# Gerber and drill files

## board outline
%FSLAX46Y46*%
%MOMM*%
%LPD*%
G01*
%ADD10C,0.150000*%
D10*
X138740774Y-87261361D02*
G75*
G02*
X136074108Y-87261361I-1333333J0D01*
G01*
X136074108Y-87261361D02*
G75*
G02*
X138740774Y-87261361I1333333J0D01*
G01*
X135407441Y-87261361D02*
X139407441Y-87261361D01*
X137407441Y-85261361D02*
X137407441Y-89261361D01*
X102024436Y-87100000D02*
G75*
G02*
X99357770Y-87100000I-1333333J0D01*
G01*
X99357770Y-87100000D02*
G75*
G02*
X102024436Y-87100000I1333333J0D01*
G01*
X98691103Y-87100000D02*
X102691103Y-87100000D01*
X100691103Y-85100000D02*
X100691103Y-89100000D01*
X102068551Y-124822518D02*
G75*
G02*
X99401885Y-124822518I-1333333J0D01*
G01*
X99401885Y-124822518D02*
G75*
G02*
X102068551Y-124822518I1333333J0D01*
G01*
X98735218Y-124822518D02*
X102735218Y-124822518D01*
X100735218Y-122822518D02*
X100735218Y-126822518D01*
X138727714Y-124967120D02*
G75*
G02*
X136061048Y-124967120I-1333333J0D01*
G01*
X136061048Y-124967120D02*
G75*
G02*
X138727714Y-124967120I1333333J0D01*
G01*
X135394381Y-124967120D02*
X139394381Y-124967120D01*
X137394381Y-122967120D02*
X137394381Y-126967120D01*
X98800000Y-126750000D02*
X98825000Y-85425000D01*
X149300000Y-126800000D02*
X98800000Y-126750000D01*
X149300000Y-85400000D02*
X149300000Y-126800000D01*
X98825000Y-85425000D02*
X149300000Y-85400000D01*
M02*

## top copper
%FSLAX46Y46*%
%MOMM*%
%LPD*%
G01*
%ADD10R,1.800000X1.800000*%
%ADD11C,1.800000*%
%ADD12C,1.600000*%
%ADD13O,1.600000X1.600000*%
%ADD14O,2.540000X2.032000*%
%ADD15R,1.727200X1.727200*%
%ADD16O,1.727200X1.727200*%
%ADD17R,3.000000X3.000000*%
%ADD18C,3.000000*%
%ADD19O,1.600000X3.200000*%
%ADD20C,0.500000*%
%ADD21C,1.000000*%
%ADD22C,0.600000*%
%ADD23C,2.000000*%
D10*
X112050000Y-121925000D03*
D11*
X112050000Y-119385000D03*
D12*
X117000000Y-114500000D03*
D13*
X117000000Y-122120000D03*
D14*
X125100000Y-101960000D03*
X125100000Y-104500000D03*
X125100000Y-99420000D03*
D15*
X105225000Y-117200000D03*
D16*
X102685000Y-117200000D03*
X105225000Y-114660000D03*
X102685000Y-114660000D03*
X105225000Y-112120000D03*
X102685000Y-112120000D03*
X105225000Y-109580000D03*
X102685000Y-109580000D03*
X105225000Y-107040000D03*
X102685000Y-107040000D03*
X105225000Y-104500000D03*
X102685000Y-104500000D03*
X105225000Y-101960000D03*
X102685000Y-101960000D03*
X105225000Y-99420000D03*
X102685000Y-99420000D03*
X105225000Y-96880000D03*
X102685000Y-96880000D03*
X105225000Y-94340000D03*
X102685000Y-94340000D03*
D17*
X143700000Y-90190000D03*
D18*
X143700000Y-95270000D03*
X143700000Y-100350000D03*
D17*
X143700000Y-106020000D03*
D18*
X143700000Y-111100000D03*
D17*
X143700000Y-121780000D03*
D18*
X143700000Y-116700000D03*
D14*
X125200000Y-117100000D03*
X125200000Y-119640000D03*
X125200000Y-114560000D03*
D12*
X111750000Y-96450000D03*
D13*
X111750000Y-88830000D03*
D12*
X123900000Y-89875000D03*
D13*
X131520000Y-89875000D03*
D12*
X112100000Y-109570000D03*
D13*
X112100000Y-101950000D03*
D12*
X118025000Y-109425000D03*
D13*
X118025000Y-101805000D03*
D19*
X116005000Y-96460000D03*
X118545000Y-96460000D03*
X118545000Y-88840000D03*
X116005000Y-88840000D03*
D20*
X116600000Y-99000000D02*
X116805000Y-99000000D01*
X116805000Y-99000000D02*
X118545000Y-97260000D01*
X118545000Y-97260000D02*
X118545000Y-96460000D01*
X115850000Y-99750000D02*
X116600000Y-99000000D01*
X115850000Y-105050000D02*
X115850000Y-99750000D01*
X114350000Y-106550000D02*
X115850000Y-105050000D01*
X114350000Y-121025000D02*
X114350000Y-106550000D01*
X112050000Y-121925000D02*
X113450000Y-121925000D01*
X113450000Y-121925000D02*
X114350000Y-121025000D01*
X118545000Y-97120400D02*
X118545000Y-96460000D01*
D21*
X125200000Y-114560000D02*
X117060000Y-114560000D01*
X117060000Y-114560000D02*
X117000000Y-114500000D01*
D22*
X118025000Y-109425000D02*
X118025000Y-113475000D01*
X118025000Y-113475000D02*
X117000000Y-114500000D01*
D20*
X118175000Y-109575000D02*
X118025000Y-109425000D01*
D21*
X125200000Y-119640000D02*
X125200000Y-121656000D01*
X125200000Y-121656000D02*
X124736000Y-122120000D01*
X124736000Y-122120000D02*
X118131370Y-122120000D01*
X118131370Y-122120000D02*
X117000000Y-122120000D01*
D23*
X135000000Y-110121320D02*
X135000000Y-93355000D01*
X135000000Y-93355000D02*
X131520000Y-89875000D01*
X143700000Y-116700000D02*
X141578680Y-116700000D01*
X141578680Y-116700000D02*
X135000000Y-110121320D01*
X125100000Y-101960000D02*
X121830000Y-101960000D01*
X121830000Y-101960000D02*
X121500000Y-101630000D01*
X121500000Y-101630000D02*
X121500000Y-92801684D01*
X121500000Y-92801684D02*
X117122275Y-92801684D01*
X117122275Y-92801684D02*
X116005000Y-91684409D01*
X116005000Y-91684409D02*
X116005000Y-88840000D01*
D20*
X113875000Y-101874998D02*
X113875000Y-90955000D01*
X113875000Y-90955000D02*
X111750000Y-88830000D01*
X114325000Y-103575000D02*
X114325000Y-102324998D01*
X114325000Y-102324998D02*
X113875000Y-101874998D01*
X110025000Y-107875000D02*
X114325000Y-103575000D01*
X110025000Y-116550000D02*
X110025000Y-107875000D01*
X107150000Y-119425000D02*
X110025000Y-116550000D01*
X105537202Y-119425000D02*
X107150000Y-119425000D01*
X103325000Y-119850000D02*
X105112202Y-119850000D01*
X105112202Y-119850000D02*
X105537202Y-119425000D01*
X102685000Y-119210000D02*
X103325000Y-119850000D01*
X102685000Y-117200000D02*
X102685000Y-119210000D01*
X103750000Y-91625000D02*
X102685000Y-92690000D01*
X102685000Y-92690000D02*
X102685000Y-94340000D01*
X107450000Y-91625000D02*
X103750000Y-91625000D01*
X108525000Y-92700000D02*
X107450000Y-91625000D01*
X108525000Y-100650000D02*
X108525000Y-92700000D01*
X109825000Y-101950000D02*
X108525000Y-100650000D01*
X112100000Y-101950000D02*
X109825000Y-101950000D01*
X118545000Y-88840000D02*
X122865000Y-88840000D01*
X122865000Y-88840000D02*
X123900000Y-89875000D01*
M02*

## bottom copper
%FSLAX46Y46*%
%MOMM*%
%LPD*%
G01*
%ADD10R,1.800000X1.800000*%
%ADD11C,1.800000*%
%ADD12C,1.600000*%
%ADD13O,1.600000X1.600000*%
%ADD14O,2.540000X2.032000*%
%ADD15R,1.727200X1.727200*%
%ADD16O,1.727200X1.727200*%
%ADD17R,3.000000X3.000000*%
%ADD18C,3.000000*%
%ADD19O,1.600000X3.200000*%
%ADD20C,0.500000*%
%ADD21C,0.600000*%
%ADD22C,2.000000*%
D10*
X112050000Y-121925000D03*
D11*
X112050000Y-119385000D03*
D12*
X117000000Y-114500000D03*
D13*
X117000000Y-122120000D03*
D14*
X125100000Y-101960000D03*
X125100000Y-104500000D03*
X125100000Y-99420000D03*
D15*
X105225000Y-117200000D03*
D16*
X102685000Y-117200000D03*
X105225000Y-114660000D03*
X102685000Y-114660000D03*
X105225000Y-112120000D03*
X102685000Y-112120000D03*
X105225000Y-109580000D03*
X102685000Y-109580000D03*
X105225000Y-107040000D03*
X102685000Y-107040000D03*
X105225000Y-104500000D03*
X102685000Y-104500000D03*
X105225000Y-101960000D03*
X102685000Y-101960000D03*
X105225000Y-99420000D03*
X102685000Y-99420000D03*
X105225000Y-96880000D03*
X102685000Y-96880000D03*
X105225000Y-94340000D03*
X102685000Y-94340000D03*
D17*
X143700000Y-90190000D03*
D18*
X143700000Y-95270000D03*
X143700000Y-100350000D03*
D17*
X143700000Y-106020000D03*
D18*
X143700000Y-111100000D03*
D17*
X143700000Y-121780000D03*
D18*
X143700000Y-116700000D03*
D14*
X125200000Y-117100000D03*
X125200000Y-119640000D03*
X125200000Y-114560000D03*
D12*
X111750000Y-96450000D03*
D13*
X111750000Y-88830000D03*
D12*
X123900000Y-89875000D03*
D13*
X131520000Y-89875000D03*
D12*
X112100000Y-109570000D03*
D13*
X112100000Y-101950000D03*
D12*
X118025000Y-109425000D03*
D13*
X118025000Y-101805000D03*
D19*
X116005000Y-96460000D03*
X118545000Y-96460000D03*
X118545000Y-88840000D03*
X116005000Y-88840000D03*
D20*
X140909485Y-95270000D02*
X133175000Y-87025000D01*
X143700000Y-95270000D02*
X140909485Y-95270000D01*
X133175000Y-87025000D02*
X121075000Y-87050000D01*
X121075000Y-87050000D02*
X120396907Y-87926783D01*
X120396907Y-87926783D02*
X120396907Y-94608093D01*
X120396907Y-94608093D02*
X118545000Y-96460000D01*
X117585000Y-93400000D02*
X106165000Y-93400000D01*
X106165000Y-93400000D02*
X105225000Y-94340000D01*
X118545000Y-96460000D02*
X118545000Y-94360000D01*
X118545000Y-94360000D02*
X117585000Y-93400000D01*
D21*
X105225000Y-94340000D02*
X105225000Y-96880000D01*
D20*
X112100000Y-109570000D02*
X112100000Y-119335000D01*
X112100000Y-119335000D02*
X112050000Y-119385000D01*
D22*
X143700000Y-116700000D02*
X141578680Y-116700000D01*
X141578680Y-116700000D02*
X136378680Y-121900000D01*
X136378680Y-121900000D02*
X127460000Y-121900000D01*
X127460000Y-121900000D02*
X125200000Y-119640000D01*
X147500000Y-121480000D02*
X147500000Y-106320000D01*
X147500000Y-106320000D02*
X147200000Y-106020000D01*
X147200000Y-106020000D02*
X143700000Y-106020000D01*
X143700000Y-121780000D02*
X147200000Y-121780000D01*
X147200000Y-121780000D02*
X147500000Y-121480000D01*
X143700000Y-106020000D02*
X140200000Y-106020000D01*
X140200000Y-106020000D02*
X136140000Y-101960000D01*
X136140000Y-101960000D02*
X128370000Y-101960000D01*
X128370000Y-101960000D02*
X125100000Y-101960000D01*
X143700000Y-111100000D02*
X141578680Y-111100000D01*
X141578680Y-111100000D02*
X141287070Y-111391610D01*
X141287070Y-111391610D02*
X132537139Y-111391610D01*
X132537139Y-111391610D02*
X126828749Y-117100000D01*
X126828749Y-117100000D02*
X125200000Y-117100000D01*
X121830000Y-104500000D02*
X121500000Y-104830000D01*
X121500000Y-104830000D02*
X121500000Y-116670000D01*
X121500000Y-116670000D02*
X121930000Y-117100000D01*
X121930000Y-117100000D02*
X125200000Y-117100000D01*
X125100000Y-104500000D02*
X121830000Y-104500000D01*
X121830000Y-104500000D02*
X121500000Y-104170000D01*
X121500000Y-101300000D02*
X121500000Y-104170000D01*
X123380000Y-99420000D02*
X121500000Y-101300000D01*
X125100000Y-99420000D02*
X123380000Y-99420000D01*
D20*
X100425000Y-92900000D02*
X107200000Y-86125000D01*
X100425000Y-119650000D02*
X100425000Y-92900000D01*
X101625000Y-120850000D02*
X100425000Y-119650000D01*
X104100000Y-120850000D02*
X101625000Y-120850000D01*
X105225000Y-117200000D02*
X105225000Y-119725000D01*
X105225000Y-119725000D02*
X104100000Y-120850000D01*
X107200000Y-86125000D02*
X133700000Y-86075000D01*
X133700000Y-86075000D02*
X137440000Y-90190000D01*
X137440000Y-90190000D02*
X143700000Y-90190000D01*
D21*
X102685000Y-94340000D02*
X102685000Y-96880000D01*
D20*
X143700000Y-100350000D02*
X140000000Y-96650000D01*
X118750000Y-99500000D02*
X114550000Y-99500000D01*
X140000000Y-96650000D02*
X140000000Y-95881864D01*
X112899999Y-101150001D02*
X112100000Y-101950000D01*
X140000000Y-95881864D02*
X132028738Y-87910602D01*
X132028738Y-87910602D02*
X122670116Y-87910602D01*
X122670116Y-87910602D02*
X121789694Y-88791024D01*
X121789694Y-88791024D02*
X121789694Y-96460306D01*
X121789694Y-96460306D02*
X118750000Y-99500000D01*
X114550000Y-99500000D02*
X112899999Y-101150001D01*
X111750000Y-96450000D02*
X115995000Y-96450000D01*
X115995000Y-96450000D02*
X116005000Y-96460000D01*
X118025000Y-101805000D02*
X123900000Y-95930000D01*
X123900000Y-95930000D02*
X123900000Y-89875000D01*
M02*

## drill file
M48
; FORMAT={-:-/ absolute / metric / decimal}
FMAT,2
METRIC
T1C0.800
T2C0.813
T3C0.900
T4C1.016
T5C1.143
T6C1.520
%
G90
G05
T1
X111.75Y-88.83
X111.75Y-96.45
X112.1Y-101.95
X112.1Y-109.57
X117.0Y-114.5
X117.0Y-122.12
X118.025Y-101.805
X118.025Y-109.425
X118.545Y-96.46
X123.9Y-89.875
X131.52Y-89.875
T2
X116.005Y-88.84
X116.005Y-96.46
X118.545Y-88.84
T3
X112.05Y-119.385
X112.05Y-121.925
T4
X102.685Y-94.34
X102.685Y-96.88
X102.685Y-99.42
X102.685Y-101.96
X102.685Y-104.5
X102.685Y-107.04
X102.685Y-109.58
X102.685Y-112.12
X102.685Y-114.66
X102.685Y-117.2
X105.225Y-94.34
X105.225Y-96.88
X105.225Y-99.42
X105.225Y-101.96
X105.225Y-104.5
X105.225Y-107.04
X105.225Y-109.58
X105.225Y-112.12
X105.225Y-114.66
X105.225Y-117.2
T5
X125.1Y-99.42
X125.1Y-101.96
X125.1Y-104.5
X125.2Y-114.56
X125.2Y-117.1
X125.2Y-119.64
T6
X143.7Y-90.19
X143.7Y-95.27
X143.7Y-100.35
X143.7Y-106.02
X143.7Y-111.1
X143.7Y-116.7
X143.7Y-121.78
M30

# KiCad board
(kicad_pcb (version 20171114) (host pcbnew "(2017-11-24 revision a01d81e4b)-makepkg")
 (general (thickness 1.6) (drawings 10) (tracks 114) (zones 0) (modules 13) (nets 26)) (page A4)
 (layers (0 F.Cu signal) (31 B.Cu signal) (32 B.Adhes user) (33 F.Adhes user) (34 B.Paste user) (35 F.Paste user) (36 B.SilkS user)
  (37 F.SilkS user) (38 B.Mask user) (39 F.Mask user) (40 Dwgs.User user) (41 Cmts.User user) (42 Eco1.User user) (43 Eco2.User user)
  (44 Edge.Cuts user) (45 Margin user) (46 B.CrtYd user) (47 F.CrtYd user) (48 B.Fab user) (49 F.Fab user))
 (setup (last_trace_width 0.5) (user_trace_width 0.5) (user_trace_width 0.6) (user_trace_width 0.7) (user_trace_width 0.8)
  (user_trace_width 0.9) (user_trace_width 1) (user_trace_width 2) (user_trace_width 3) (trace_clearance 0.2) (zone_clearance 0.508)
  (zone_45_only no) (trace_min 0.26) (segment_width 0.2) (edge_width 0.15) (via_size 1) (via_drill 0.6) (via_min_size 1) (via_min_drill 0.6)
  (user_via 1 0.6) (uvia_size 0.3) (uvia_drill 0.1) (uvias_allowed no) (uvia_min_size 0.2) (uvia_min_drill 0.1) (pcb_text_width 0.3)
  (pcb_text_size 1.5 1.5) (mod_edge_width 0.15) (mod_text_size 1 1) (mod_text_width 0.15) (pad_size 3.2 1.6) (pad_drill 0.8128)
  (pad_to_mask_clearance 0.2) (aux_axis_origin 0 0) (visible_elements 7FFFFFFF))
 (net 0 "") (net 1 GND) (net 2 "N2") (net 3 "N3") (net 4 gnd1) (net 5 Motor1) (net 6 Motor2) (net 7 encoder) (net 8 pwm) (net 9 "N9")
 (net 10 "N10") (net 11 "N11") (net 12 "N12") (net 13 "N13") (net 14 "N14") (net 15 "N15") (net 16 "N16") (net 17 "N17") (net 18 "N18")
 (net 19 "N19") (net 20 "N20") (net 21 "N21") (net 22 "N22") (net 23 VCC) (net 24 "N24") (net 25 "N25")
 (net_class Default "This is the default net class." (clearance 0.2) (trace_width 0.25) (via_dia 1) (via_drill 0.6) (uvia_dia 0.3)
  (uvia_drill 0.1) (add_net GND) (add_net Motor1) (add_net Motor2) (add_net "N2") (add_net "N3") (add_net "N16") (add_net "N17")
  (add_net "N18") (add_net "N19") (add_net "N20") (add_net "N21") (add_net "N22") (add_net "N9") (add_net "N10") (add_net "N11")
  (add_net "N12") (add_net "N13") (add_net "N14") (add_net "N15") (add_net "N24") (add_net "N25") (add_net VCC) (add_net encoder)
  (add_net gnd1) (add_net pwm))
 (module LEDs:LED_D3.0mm (layer F.Cu) (at 112.05 121.925 90)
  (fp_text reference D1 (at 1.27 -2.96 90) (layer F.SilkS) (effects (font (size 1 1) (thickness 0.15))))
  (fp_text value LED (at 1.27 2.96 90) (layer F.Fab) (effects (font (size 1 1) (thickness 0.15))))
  (pad 1 thru_hole rect (at 0 0 90) (size 1.8 1.8) (drill 0.9) (layers *.Cu *.Mask) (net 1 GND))
  (pad 2 thru_hole circle (at 2.54 0 90) (size 1.8 1.8) (drill 0.9) (layers *.Cu *.Mask) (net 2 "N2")))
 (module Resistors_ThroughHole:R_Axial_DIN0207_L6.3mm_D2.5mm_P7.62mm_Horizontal (layer F.Cu) (at 117 114.5 270)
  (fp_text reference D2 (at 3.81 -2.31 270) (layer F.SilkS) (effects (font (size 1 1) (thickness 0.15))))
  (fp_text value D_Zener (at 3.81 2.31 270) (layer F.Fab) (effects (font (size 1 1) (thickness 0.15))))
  (pad 1 thru_hole circle (at 0 0 270) (size 1.6 1.6) (drill 0.8) (layers *.Cu *.Mask) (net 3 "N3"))
  (pad 2 thru_hole oval (at 7.62 0 270) (size 1.6 1.6) (drill 0.8) (layers *.Cu *.Mask) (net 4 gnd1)))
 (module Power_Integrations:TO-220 (layer F.Cu) (at 125.1 101.96 270)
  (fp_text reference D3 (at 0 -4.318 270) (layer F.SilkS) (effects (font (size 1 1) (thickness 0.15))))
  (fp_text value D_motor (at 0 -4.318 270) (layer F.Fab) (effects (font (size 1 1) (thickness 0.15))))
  (pad 2 thru_hole oval (at 0 0 270) (size 2.032 2.54) (drill 1.143) (layers *.Cu *.Mask) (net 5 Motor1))
  (pad 3 thru_hole oval (at 2.54 0 270) (size 2.032 2.54) (drill 1.143) (layers *.Cu *.Mask) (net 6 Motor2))
  (pad 1 thru_hole oval (at -2.54 0 270) (size 2.032 2.54) (drill 1.143) (layers *.Cu *.Mask) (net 6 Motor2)))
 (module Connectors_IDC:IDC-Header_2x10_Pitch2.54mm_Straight (layer F.Cu) (at 105.225 117.2 180)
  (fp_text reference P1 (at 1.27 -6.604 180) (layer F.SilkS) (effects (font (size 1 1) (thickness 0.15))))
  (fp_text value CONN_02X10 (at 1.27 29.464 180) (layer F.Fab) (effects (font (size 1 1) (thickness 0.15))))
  (pad 1 thru_hole rect (at 0 0 180) (size 1.7272 1.7272) (drill 1.016) (layers *.Cu *.Mask) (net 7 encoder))
  (pad 2 thru_hole oval (at 2.54 0 180) (size 1.7272 1.7272) (drill 1.016) (layers *.Cu *.Mask) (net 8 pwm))
  (pad 3 thru_hole oval (at 0 2.54 180) (size 1.7272 1.7272) (drill 1.016) (layers *.Cu *.Mask) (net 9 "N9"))
  (pad 4 thru_hole oval (at 2.54 2.54 180) (size 1.7272 1.7272) (drill 1.016) (layers *.Cu *.Mask) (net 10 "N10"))
  (pad 5 thru_hole oval (at 0 5.08 180) (size 1.7272 1.7272) (drill 1.016) (layers *.Cu *.Mask) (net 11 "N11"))
  (pad 6 thru_hole oval (at 2.54 5.08 180) (size 1.7272 1.7272) (drill 1.016) (layers *.Cu *.Mask) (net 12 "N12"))
  (pad 7 thru_hole oval (at 0 7.62 180) (size 1.7272 1.7272) (drill 1.016) (layers *.Cu *.Mask) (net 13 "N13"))
  (pad 8 thru_hole oval (at 2.54 7.62 180) (size 1.7272 1.7272) (drill 1.016) (layers *.Cu *.Mask) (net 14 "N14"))
  (pad 9 thru_hole oval (at 0 10.16 180) (size 1.7272 1.7272) (drill 1.016) (layers *.Cu *.Mask) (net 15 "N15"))
  (pad 10 thru_hole oval (at 2.54 10.16 180) (size 1.7272 1.7272) (drill 1.016) (layers *.Cu *.Mask) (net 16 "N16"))
  (pad 11 thru_hole oval (at 0 12.7 180) (size 1.7272 1.7272) (drill 1.016) (layers *.Cu *.Mask) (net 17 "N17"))
  (pad 12 thru_hole oval (at 2.54 12.7 180) (size 1.7272 1.7272) (drill 1.016) (layers *.Cu *.Mask) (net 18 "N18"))
  (pad 13 thru_hole oval (at 0 15.24 180) (size 1.7272 1.7272) (drill 1.016) (layers *.Cu *.Mask) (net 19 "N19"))
  (pad 14 thru_hole oval (at 2.54 15.24 180) (size 1.7272 1.7272) (drill 1.016) (layers *.Cu *.Mask) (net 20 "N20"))
  (pad 15 thru_hole oval (at 0 17.78 180) (size 1.7272 1.7272) (drill 1.016) (layers *.Cu *.Mask) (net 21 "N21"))
  (pad 16 thru_hole oval (at 2.54 17.78 180) (size 1.7272 1.7272) (drill 1.016) (layers *.Cu *.Mask) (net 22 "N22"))
  (pad 17 thru_hole oval (at 0 20.32 180) (size 1.7272 1.7272) (drill 1.016) (layers *.Cu *.Mask) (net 1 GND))
  (pad 18 thru_hole oval (at 2.54 20.32 180) (size 1.7272 1.7272) (drill 1.016) (layers *.Cu *.Mask) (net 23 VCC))
  (pad 19 thru_hole oval (at 0 22.86 180) (size 1.7272 1.7272) (drill 1.016) (layers *.Cu *.Mask) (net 1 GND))
  (pad 20 thru_hole oval (at 2.54 22.86 180) (size 1.7272 1.7272) (drill 1.016) (layers *.Cu *.Mask) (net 23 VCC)))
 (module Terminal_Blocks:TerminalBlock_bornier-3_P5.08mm (layer F.Cu) (at 143.7 90.19 270)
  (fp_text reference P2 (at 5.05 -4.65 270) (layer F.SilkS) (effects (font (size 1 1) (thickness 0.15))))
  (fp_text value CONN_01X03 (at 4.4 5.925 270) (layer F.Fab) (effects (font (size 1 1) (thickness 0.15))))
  (pad 1 thru_hole rect (at 0 0 270) (size 3 3) (drill 1.52) (layers *.Cu *.Mask) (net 7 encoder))
  (pad 2 thru_hole circle (at 5.08 0 270) (size 3 3) (drill 1.52) (layers *.Cu *.Mask) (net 1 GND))
  (pad 3 thru_hole circle (at 10.16 0 270) (size 3 3) (drill 1.52) (layers *.Cu *.Mask) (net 23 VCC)))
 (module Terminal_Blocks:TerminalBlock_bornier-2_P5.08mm (layer F.Cu) (at 143.7 106.02 270)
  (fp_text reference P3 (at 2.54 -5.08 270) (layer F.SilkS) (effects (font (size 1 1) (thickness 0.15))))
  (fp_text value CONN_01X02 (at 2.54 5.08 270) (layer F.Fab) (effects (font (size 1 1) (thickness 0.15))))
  (pad 1 thru_hole rect (at 0 0 270) (size 3 3) (drill 1.52) (layers *.Cu *.Mask) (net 5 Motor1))
  (pad 2 thru_hole circle (at 5.08 0 270) (size 3 3) (drill 1.52) (layers *.Cu *.Mask) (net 6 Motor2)))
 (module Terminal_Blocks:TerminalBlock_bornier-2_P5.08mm (layer F.Cu) (at 143.7 121.78 90)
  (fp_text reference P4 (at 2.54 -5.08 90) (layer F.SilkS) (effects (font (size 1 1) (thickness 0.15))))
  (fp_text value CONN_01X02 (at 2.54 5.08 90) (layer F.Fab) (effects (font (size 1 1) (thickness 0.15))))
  (pad 1 thru_hole rect (at 0 0 90) (size 3 3) (drill 1.52) (layers *.Cu *.Mask) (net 5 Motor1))
  (pad 2 thru_hole circle (at 5.08 0 90) (size 3 3) (drill 1.52) (layers *.Cu *.Mask) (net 4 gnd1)))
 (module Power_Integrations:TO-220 (layer F.Cu) (at 125.2 117.1 270)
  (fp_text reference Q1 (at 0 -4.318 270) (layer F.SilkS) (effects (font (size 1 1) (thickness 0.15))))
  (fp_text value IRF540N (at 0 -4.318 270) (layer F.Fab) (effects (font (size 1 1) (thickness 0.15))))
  (pad 2 thru_hole oval (at 0 0 270) (size 2.032 2.54) (drill 1.143) (layers *.Cu *.Mask) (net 6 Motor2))
  (pad 3 thru_hole oval (at 2.54 0 270) (size 2.032 2.54) (drill 1.143) (layers *.Cu *.Mask) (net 4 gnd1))
  (pad 1 thru_hole oval (at -2.54 0 270) (size 2.032 2.54) (drill 1.143) (layers *.Cu *.Mask) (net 3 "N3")))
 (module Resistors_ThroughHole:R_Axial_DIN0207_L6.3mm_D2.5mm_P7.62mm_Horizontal (layer F.Cu) (at 111.75 96.45 90)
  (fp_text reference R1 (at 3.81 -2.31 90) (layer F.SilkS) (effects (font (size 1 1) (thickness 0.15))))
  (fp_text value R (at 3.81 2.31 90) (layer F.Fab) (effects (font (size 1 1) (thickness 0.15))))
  (pad 1 thru_hole circle (at 0 0 90) (size 1.6 1.6) (drill 0.8) (layers *.Cu *.Mask) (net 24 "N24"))
  (pad 2 thru_hole oval (at 7.62 0 90) (size 1.6 1.6) (drill 0.8) (layers *.Cu *.Mask) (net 8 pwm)))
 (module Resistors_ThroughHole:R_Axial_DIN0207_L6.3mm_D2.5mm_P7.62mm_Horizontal (layer F.Cu) (at 123.9 89.875)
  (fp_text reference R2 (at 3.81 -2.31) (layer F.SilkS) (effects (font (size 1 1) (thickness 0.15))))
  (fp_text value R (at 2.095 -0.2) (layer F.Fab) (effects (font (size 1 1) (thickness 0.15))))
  (pad 1 thru_hole circle (at 0 0) (size 1.6 1.6) (drill 0.8) (layers *.Cu *.Mask) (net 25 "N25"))
  (pad 2 thru_hole oval (at 7.62 0) (size 1.6 1.6) (drill 0.8) (layers *.Cu *.Mask) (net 4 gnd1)))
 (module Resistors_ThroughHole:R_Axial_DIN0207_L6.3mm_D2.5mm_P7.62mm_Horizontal (layer F.Cu) (at 112.1 109.57 90)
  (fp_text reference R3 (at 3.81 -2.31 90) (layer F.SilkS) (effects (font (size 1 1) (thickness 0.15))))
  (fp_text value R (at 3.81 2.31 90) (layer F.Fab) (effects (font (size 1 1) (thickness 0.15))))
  (pad 1 thru_hole circle (at 0 0 90) (size 1.6 1.6) (drill 0.8) (layers *.Cu *.Mask) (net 2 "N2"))
  (pad 2 thru_hole oval (at 7.62 0 90) (size 1.6 1.6) (drill 0.8) (layers *.Cu *.Mask) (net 23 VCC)))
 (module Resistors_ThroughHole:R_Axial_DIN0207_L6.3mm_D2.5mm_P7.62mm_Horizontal (layer F.Cu) (at 118.025 109.425 90)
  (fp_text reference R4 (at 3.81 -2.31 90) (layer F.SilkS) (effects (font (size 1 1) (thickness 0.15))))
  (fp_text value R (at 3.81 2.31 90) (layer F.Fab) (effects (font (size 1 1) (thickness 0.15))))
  (pad 1 thru_hole circle (at 0 0 90) (size 1.6 1.6) (drill 0.8) (layers *.Cu *.Mask) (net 3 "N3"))
  (pad 2 thru_hole oval (at 7.62 0 90) (size 1.6 1.6) (drill 0.8) (layers *.Cu *.Mask) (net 25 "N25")))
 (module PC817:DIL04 (layer F.Cu) (at 117.275 92.65) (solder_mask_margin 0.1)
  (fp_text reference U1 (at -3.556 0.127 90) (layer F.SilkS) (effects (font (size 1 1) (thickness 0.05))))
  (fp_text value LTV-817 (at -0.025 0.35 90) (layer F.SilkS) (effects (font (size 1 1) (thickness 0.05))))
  (pad 1 thru_hole oval (at -1.27 3.81 270) (size 3.2 1.6) (drill 0.8128) (layers *.Cu *.Mask F.SilkS) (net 24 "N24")
   (solder_mask_margin 0.2))
  (pad 2 thru_hole oval (at 1.27 3.81 270) (size 3.2 1.6) (drill 0.8) (layers *.Cu *.Mask F.SilkS) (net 1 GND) (solder_mask_margin 0.2))
  (pad 3 thru_hole oval (at 1.27 -3.81 90) (size 3.2 1.6) (drill 0.8128) (layers *.Cu *.Mask F.SilkS) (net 25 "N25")
   (solder_mask_margin 0.2))
  (pad 4 thru_hole oval (at -1.27 -3.81 90) (size 3.2 1.6) (drill 0.8128) (layers *.Cu *.Mask F.SilkS) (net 5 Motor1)
   (solder_mask_margin 0.2)))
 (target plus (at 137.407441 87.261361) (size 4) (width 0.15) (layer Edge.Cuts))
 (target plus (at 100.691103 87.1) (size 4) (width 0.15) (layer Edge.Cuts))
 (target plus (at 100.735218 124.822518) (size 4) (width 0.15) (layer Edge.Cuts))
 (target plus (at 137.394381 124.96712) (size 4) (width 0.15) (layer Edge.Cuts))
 (gr_line (start 98.8 126.75) (end 98.825 85.425) (layer Edge.Cuts) (width 0.15))
 (gr_line (start 149.3 126.8) (end 98.8 126.75) (layer Edge.Cuts) (width 0.15))
 (gr_line (start 149.3 85.4) (end 149.3 126.8) (layer Edge.Cuts) (width 0.15))
 (gr_line (start 98.825 85.425) (end 149.3 85.4) (layer Edge.Cuts) (width 0.15))
 (segment (start 140.909485 95.27) (end 133.175 87.025) (width 0.5) (layer B.Cu) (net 1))
 (segment (start 143.7 95.27) (end 140.909485 95.27) (width 0.5) (layer B.Cu) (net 1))
 (segment (start 133.175 87.025) (end 121.075 87.05) (width 0.5) (layer B.Cu) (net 1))
 (segment (start 121.075 87.05) (end 120.396907 87.926783) (width 0.5) (layer B.Cu) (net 1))
 (segment (start 120.396907 87.926783) (end 120.396907 94.608093) (width 0.5) (layer B.Cu) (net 1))
 (segment (start 120.396907 94.608093) (end 118.545 96.46) (width 0.5) (layer B.Cu) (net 1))
 (segment (start 116.6 99) (end 116.805 99) (width 0.5) (layer F.Cu) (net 1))
 (segment (start 116.805 99) (end 118.545 97.26) (width 0.5) (layer F.Cu) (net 1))
 (segment (start 118.545 97.26) (end 118.545 96.46) (width 0.5) (layer F.Cu) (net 1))
 (segment (start 115.85 99.75) (end 116.6 99) (width 0.5) (layer F.Cu) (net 1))
 (segment (start 115.85 105.05) (end 115.85 99.75) (width 0.5) (layer F.Cu) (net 1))
 (segment (start 114.35 106.55) (end 115.85 105.05) (width 0.5) (layer F.Cu) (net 1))
 (segment (start 114.35 121.025) (end 114.35 106.55) (width 0.5) (layer F.Cu) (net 1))
 (segment (start 112.05 121.925) (end 113.45 121.925) (width 0.5) (layer F.Cu) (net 1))
 (segment (start 113.45 121.925) (end 114.35 121.025) (width 0.5) (layer F.Cu) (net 1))
 (segment (start 117.585 93.4) (end 106.165 93.4) (width 0.5) (layer B.Cu) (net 1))
 (segment (start 106.165 93.4) (end 105.225 94.34) (width 0.5) (layer B.Cu) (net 1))
 (segment (start 118.545 96.46) (end 118.545 94.36) (width 0.5) (layer B.Cu) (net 1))
 (segment (start 118.545 94.36) (end 117.585 93.4) (width 0.5) (layer B.Cu) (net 1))
 (segment (start 105.225 94.34) (end 105.225 96.88) (width 0.6) (layer B.Cu) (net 1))
 (segment (start 118.545 97.1204) (end 118.545 96.46) (width 0.5) (layer F.Cu) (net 1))
 (segment (start 112.1 109.57) (end 112.1 119.335) (width 0.5) (layer B.Cu) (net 2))
 (segment (start 112.1 119.335) (end 112.05 119.385) (width 0.5) (layer B.Cu) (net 2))
 (segment (start 125.2 114.56) (end 117.06 114.56) (width 1) (layer F.Cu) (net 3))
 (segment (start 117.06 114.56) (end 117 114.5) (width 1) (layer F.Cu) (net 3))
 (segment (start 118.025 109.425) (end 118.025 113.475) (width 0.6) (layer F.Cu) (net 3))
 (segment (start 118.025 113.475) (end 117 114.5) (width 0.6) (layer F.Cu) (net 3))
 (segment (start 118.175 109.575) (end 118.025 109.425) (width 0.5) (layer F.Cu) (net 3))
 (segment (start 125.2 119.64) (end 125.2 121.656) (width 1) (layer F.Cu) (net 4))
 (segment (start 125.2 121.656) (end 124.736 122.12) (width 1) (layer F.Cu) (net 4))
 (segment (start 124.736 122.12) (end 118.13137 122.12) (width 1) (layer F.Cu) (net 4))
 (segment (start 118.13137 122.12) (end 117 122.12) (width 1) (layer F.Cu) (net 4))
 (segment (start 135 110.12132) (end 135 93.355) (width 2) (layer F.Cu) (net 4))
 (segment (start 135 93.355) (end 131.52 89.875) (width 2) (layer F.Cu) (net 4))
 (segment (start 143.7 116.7) (end 141.57868 116.7) (width 2) (layer F.Cu) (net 4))
 (segment (start 141.57868 116.7) (end 135 110.12132) (width 2) (layer F.Cu) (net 4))
 (segment (start 143.7 116.7) (end 141.57868 116.7) (width 2) (layer B.Cu) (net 4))
 (segment (start 141.57868 116.7) (end 136.37868 121.9) (width 2) (layer B.Cu) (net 4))
 (segment (start 136.37868 121.9) (end 127.46 121.9) (width 2) (layer B.Cu) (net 4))
 (segment (start 127.46 121.9) (end 125.2 119.64) (width 2) (layer B.Cu) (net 4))
 (segment (start 125.1 101.96) (end 121.83 101.96) (width 2) (layer F.Cu) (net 5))
 (segment (start 121.83 101.96) (end 121.5 101.63) (width 2) (layer F.Cu) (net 5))
 (segment (start 121.5 101.63) (end 121.5 92.801684) (width 2) (layer F.Cu) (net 5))
 (segment (start 121.5 92.801684) (end 117.122275 92.801684) (width 2) (layer F.Cu) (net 5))
 (segment (start 117.122275 92.801684) (end 116.005 91.684409) (width 2) (layer F.Cu) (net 5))
 (segment (start 116.005 91.684409) (end 116.005 88.84) (width 2) (layer F.Cu) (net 5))
 (segment (start 147.5 121.48) (end 147.5 106.32) (width 2) (layer B.Cu) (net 5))
 (segment (start 147.5 106.32) (end 147.2 106.02) (width 2) (layer B.Cu) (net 5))
 (segment (start 147.2 106.02) (end 143.7 106.02) (width 2) (layer B.Cu) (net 5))
 (segment (start 143.7 121.78) (end 147.2 121.78) (width 2) (layer B.Cu) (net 5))
 (segment (start 147.2 121.78) (end 147.5 121.48) (width 2) (layer B.Cu) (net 5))
 (segment (start 143.7 106.02) (end 140.2 106.02) (width 2) (layer B.Cu) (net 5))
 (segment (start 140.2 106.02) (end 136.14 101.96) (width 2) (layer B.Cu) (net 5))
 (segment (start 136.14 101.96) (end 128.37 101.96) (width 2) (layer B.Cu) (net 5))
 (segment (start 128.37 101.96) (end 125.1 101.96) (width 2) (layer B.Cu) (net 5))
 (segment (start 143.7 111.1) (end 141.57868 111.1) (width 2) (layer B.Cu) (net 6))
 (segment (start 141.57868 111.1) (end 141.28707 111.39161) (width 2) (layer B.Cu) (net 6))
 (segment (start 141.28707 111.39161) (end 132.537139 111.39161) (width 2) (layer B.Cu) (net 6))
 (segment (start 132.537139 111.39161) (end 126.828749 117.1) (width 2) (layer B.Cu) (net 6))
 (segment (start 126.828749 117.1) (end 125.2 117.1) (width 2) (layer B.Cu) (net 6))
 (segment (start 121.83 104.5) (end 121.5 104.83) (width 2) (layer B.Cu) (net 6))
 (segment (start 121.5 104.83) (end 121.5 116.67) (width 2) (layer B.Cu) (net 6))
 (segment (start 121.5 116.67) (end 121.93 117.1) (width 2) (layer B.Cu) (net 6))
 (segment (start 121.93 117.1) (end 125.2 117.1) (width 2) (layer B.Cu) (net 6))
 (segment (start 125.1 104.5) (end 121.83 104.5) (width 2) (layer B.Cu) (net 6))
 (segment (start 121.83 104.5) (end 121.5 104.17) (width 2) (layer B.Cu) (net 6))
 (segment (start 121.5 101.3) (end 121.5 104.17) (width 2) (layer B.Cu) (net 6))
 (segment (start 123.38 99.42) (end 121.5 101.3) (width 2) (layer B.Cu) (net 6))
 (segment (start 125.1 99.42) (end 123.38 99.42) (width 2) (layer B.Cu) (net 6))
 (segment (start 100.425 92.9) (end 107.2 86.125) (width 0.5) (layer B.Cu) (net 7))
 (segment (start 100.425 119.65) (end 100.425 92.9) (width 0.5) (layer B.Cu) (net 7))
 (segment (start 101.625 120.85) (end 100.425 119.65) (width 0.5) (layer B.Cu) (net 7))
 (segment (start 104.1 120.85) (end 101.625 120.85) (width 0.5) (layer B.Cu) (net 7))
 (segment (start 105.225 117.2) (end 105.225 119.725) (width 0.5) (layer B.Cu) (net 7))
 (segment (start 105.225 119.725) (end 104.1 120.85) (width 0.5) (layer B.Cu) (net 7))
 (segment (start 107.2 86.125) (end 133.7 86.075) (width 0.5) (layer B.Cu) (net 7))
 (segment (start 133.7 86.075) (end 137.44 90.19) (width 0.5) (layer B.Cu) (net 7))
 (segment (start 137.44 90.19) (end 143.7 90.19) (width 0.5) (layer B.Cu) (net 7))
 (segment (start 113.875 101.874998) (end 113.875 90.955) (width 0.5) (layer F.Cu) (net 8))
 (segment (start 113.875 90.955) (end 111.75 88.83) (width 0.5) (layer F.Cu) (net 8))
 (segment (start 114.325 103.575) (end 114.325 102.324998) (width 0.5) (layer F.Cu) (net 8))
 (segment (start 114.325 102.324998) (end 113.875 101.874998) (width 0.5) (layer F.Cu) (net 8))
 (segment (start 110.025 107.875) (end 114.325 103.575) (width 0.5) (layer F.Cu) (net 8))
 (segment (start 110.025 116.55) (end 110.025 107.875) (width 0.5) (layer F.Cu) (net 8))
 (segment (start 107.15 119.425) (end 110.025 116.55) (width 0.5) (layer F.Cu) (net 8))
 (segment (start 105.537202 119.425) (end 107.15 119.425) (width 0.5) (layer F.Cu) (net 8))
 (segment (start 103.325 119.85) (end 105.112202 119.85) (width 0.5) (layer F.Cu) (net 8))
 (segment (start 105.112202 119.85) (end 105.537202 119.425) (width 0.5) (layer F.Cu) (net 8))
 (segment (start 102.685 119.21) (end 103.325 119.85) (width 0.5) (layer F.Cu) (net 8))
 (segment (start 102.685 117.2) (end 102.685 119.21) (width 0.5) (layer F.Cu) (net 8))
 (segment (start 103.75 91.625) (end 102.685 92.69) (width 0.5) (layer F.Cu) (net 23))
 (segment (start 102.685 92.69) (end 102.685 94.34) (width 0.5) (layer F.Cu) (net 23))
 (segment (start 107.45 91.625) (end 103.75 91.625) (width 0.5) (layer F.Cu) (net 23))
 (segment (start 108.525 92.7) (end 107.45 91.625) (width 0.5) (layer F.Cu) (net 23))
 (segment (start 108.525 100.65) (end 108.525 92.7) (width 0.5) (layer F.Cu) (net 23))
 (segment (start 109.825 101.95) (end 108.525 100.65) (width 0.5) (layer F.Cu) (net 23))
 (segment (start 112.1 101.95) (end 109.825 101.95) (width 0.5) (layer F.Cu) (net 23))
 (segment (start 102.685 94.34) (end 102.685 96.88) (width 0.6) (layer B.Cu) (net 23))
 (segment (start 143.7 100.35) (end 140 96.65) (width 0.5) (layer B.Cu) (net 23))
 (segment (start 118.75 99.5) (end 114.55 99.5) (width 0.5) (layer B.Cu) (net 23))
 (segment (start 140 96.65) (end 140 95.881864) (width 0.5) (layer B.Cu) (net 23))
 (segment (start 112.899999 101.150001) (end 112.1 101.95) (width 0.5) (layer B.Cu) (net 23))
 (segment (start 140 95.881864) (end 132.028738 87.910602) (width 0.5) (layer B.Cu) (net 23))
 (segment (start 132.028738 87.910602) (end 122.670116 87.910602) (width 0.5) (layer B.Cu) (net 23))
 (segment (start 122.670116 87.910602) (end 121.789694 88.791024) (width 0.5) (layer B.Cu) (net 23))
 (segment (start 121.789694 88.791024) (end 121.789694 96.460306) (width 0.5) (layer B.Cu) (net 23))
 (segment (start 121.789694 96.460306) (end 118.75 99.5) (width 0.5) (layer B.Cu) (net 23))
 (segment (start 114.55 99.5) (end 112.899999 101.150001) (width 0.5) (layer B.Cu) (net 23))
 (segment (start 111.75 96.45) (end 115.995 96.45) (width 0.5) (layer B.Cu) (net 24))
 (segment (start 115.995 96.45) (end 116.005 96.46) (width 0.5) (layer B.Cu) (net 24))
 (segment (start 118.025 101.805) (end 123.9 95.93) (width 0.5) (layer B.Cu) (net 25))
 (segment (start 123.9 95.93) (end 123.9 89.875) (width 0.5) (layer B.Cu) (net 25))
 (segment (start 118.545 88.84) (end 122.865 88.84) (width 0.5) (layer F.Cu) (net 25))
 (segment (start 122.865 88.84) (end 123.9 89.875) (width 0.5) (layer F.Cu) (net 25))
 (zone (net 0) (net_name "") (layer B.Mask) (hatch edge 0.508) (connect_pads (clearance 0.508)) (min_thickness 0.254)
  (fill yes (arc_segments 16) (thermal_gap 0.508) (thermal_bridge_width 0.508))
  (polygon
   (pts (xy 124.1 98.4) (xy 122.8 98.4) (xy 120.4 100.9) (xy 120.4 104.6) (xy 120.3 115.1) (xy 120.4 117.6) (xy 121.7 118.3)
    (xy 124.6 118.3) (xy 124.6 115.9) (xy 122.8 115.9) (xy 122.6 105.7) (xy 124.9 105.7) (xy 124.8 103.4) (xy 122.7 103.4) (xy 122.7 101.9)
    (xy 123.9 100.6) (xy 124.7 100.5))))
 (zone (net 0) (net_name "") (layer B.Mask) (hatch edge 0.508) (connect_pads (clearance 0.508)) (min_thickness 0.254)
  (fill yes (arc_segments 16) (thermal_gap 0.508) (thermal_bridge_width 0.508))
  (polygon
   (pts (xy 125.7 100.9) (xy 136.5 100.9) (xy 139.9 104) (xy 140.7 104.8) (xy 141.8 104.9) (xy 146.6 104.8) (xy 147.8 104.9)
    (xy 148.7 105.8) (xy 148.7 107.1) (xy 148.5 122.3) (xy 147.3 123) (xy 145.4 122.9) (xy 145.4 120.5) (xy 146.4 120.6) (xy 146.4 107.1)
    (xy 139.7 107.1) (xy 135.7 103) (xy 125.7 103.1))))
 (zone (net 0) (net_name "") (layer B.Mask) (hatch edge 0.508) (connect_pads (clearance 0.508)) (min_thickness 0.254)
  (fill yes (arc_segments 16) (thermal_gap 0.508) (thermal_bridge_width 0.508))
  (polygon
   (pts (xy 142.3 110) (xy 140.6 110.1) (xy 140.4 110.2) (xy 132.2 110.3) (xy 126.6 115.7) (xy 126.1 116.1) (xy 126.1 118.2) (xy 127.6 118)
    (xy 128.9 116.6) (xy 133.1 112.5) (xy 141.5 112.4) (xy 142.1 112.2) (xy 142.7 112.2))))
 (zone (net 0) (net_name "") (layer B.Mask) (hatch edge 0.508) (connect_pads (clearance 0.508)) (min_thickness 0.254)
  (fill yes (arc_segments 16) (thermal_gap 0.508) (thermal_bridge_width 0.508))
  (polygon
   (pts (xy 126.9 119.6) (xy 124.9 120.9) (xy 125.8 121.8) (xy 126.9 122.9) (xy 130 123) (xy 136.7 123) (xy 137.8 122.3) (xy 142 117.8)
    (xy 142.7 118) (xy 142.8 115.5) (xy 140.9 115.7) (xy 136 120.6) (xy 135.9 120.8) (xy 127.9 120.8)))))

